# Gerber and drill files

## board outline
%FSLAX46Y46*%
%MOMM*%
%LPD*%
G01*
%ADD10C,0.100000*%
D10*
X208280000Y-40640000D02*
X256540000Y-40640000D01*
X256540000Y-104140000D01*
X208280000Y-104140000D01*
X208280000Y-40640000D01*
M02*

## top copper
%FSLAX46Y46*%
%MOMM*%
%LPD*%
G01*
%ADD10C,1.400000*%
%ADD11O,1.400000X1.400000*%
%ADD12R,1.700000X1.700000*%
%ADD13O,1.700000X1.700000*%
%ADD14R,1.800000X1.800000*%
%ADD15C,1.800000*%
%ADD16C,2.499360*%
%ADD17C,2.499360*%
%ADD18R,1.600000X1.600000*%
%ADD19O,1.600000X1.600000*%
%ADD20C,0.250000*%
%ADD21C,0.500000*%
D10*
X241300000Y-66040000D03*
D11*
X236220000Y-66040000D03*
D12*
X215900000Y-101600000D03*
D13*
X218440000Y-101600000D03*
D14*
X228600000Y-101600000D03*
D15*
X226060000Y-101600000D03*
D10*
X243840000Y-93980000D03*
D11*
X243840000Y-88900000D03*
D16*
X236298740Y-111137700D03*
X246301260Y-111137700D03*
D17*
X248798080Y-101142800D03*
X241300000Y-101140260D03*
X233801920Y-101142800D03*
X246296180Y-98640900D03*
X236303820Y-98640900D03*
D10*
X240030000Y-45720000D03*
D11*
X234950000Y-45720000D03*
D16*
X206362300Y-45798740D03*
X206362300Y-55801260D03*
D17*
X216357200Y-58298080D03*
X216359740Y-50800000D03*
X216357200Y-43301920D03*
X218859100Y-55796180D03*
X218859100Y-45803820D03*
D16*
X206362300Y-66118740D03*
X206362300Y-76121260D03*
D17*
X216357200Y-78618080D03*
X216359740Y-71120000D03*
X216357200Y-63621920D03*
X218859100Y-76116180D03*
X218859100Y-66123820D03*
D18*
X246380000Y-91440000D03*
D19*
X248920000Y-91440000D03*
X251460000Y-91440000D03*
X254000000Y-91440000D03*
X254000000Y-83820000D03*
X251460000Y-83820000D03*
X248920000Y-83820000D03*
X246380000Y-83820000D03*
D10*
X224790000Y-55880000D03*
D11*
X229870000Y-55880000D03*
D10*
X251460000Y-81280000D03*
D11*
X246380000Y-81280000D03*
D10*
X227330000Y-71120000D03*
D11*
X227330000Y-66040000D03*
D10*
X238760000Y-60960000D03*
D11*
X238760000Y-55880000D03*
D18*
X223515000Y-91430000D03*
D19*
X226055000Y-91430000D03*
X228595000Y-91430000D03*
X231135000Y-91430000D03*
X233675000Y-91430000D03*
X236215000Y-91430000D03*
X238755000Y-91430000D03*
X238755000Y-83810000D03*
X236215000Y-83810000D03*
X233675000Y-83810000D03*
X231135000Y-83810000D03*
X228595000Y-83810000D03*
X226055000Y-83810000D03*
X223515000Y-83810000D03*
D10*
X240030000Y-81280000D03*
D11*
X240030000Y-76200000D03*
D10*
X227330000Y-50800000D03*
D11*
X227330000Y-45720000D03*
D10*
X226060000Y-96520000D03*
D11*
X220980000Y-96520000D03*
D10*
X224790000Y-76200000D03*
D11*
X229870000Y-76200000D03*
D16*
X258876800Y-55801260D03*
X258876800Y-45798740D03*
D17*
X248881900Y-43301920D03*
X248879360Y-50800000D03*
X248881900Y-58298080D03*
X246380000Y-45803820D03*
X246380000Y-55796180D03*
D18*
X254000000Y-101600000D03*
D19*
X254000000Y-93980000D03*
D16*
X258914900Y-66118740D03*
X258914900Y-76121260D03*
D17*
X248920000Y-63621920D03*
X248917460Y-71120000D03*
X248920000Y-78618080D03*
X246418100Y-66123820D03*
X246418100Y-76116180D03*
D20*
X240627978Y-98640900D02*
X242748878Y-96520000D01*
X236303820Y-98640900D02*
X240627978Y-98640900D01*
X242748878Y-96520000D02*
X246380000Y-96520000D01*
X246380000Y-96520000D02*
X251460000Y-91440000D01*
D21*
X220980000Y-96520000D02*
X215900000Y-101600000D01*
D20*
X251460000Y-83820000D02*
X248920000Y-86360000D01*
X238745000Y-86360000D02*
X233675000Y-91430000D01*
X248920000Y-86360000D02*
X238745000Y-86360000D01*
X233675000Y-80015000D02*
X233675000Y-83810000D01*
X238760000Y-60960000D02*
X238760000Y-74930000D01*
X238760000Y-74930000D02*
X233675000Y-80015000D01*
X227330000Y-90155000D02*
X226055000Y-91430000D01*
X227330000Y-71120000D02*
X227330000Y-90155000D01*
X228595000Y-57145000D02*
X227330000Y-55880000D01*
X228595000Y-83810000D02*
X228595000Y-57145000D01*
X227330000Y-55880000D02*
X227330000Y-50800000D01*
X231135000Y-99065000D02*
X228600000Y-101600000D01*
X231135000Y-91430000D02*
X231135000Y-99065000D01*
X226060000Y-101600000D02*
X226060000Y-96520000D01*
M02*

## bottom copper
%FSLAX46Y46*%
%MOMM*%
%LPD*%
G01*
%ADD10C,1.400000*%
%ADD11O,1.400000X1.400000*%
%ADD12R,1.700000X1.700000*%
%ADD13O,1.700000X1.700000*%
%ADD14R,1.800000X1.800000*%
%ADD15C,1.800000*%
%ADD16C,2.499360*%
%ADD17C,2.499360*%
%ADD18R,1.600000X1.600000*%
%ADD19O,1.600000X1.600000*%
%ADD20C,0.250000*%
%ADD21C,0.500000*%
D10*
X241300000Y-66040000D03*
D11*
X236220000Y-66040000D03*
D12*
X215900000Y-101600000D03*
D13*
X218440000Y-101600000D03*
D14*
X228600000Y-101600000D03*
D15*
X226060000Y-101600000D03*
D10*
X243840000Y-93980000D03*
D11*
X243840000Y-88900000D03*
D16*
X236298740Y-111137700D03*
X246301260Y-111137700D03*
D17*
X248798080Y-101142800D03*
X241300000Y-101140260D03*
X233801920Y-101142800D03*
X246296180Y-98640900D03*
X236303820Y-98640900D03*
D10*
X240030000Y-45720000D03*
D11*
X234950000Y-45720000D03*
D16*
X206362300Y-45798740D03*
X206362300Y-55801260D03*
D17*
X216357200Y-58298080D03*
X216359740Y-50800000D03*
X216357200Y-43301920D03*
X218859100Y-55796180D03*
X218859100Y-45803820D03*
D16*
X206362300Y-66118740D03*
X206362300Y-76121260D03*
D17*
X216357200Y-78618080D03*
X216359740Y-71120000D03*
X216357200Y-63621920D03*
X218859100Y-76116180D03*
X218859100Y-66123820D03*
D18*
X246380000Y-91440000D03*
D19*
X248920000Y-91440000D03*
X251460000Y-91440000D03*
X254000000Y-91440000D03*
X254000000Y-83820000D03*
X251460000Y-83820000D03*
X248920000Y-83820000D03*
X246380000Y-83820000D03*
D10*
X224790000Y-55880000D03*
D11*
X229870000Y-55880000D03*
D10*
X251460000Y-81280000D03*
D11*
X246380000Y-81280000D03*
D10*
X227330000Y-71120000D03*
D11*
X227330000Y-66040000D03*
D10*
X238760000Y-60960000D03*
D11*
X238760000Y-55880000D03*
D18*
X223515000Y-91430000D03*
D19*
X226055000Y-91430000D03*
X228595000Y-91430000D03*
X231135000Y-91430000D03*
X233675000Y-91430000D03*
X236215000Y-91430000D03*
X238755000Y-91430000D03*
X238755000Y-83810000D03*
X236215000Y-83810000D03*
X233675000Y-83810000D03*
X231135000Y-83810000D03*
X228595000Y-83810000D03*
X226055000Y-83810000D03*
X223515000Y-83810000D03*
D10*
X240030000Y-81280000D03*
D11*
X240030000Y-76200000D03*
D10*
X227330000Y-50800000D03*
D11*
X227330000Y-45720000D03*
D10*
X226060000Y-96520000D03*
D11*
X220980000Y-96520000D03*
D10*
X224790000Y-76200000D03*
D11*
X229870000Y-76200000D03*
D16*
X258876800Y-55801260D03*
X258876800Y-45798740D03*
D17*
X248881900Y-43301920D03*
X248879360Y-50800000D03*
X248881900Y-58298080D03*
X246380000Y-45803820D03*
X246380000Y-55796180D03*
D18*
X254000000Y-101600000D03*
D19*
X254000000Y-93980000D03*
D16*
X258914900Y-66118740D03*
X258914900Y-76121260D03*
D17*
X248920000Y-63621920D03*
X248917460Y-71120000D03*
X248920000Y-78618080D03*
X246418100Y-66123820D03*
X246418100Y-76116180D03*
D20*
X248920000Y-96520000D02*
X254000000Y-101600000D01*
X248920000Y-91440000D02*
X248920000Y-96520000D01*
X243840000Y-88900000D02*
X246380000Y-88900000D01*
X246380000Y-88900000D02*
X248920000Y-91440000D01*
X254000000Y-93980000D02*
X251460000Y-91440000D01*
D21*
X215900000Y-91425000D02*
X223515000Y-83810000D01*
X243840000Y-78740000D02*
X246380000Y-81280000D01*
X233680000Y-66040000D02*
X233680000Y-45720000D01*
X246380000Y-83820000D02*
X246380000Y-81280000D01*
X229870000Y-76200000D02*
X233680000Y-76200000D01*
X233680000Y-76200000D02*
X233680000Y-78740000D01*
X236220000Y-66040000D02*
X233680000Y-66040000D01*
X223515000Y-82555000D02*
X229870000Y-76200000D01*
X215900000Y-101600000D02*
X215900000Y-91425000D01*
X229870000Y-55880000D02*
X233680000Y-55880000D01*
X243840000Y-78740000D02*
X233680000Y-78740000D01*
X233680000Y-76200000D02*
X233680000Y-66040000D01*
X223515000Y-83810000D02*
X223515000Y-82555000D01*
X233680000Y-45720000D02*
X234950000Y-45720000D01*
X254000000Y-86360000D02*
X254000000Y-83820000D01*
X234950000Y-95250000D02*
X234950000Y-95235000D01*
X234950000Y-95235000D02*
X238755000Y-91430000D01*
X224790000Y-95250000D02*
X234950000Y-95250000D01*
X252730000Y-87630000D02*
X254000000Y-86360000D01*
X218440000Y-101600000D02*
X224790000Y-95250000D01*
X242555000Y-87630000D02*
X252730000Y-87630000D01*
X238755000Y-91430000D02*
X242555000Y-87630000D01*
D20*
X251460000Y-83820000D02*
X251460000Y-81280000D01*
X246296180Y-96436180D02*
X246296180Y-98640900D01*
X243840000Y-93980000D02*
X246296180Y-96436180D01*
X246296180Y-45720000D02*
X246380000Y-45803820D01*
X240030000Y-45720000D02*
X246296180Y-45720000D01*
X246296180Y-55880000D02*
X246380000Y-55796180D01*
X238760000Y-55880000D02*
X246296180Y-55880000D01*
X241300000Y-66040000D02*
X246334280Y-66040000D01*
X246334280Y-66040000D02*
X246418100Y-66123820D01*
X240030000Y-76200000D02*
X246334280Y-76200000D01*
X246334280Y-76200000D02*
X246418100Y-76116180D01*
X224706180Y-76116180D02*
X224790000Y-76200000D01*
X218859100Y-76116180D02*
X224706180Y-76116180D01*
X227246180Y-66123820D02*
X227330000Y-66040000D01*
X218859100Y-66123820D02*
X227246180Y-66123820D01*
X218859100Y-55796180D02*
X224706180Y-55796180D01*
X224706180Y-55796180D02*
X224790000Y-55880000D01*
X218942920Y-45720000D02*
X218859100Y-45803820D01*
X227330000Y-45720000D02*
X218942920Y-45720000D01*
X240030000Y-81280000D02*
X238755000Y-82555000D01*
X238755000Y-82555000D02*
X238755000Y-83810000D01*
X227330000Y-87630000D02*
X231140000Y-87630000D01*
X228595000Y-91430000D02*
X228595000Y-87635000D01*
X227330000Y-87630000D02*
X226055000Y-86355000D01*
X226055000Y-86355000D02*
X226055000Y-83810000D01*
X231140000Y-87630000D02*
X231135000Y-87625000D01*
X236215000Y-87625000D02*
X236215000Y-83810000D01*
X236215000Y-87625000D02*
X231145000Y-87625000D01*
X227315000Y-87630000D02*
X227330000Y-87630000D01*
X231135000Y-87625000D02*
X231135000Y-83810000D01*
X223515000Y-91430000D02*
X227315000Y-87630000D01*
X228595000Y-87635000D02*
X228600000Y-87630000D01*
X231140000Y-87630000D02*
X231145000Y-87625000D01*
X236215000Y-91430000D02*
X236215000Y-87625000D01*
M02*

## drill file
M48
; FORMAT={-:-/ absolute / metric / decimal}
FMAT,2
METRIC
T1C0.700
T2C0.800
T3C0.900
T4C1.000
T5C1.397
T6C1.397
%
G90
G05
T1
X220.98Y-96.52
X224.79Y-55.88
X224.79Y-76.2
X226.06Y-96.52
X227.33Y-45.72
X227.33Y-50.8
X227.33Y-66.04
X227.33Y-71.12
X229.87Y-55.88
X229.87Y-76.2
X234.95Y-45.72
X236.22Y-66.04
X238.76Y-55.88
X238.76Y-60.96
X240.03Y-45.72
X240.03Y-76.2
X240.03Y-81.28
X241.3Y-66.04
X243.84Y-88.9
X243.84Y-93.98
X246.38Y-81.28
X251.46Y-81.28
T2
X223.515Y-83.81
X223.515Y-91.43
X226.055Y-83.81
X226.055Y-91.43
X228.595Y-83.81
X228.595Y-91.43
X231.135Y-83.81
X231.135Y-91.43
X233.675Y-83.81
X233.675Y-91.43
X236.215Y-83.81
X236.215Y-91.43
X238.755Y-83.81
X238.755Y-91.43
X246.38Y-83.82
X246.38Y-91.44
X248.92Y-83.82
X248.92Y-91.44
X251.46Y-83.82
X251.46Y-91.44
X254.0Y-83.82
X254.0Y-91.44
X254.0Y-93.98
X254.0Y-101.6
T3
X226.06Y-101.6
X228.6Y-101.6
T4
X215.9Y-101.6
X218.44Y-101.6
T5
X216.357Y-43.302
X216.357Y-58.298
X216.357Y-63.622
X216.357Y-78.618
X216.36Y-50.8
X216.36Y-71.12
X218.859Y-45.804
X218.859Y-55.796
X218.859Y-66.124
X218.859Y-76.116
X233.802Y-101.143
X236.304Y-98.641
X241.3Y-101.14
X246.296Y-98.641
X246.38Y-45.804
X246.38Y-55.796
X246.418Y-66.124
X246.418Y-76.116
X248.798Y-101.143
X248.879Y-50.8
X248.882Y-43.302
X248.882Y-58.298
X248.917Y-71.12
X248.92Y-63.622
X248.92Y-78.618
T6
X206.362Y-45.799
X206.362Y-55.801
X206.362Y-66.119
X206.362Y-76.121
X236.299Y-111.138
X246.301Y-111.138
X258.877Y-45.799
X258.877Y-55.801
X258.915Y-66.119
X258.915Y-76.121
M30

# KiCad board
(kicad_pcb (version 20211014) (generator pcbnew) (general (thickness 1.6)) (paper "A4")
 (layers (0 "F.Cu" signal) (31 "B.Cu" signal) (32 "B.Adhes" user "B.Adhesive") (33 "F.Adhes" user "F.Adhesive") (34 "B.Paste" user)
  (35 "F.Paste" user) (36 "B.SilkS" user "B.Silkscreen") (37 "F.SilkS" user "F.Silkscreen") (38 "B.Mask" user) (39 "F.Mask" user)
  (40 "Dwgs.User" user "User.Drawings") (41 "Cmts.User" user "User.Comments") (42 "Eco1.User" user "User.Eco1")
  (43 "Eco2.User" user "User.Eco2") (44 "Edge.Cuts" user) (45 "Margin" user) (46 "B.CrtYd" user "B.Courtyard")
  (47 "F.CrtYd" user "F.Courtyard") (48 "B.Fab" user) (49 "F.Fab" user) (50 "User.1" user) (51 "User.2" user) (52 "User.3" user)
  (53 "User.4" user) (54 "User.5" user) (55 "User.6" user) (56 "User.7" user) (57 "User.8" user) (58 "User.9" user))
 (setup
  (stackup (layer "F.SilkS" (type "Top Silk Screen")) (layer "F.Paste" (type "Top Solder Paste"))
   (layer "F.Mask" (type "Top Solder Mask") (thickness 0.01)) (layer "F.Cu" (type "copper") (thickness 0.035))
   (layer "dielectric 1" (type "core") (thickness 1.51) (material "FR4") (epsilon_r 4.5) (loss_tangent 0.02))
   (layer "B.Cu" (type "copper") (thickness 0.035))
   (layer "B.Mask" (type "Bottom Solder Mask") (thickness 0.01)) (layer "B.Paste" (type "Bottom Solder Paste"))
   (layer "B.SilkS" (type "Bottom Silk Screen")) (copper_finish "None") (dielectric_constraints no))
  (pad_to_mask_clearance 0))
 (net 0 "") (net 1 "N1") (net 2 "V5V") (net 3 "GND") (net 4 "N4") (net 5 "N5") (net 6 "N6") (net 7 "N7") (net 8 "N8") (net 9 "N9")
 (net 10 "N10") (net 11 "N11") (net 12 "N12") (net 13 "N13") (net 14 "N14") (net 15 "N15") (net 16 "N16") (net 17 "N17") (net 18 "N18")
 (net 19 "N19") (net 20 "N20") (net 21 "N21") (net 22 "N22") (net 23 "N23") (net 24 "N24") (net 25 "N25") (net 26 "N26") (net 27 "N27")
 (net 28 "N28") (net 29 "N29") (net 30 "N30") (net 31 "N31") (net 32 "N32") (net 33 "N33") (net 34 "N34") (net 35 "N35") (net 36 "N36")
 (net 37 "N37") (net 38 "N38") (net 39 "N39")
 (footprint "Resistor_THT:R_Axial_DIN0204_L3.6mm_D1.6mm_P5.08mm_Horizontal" (layer "F.Cu") (at 241.3 66.04 180)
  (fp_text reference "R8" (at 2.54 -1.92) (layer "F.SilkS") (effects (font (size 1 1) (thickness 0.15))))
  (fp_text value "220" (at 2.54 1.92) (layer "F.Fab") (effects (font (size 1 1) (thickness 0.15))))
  (pad "1" thru_hole circle (at 0 0 180) (size 1.4 1.4) (drill 0.7) (layers *.Cu *.Mask) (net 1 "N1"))
  (pad "2" thru_hole oval (at 5.08 0 180) (size 1.4 1.4) (drill 0.7) (layers *.Cu *.Mask) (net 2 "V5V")))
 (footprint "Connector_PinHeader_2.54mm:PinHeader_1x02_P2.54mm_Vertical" (layer "F.Cu") (at 215.9 101.6 90)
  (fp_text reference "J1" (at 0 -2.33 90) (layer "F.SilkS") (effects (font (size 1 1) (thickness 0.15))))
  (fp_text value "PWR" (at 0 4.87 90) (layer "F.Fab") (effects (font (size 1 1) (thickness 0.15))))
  (pad "1" thru_hole rect (at 0 0 90) (size 1.7 1.7) (drill 1) (layers *.Cu *.Mask) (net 2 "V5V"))
  (pad "2" thru_hole oval (at 0 2.54 90) (size 1.7 1.7) (drill 1) (layers *.Cu *.Mask) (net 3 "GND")))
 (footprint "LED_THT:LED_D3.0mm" (layer "F.Cu") (at 228.6 101.6 180)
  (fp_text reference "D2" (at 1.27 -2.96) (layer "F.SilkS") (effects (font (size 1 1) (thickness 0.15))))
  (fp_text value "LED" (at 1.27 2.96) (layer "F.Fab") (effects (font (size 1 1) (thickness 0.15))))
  (pad "1" thru_hole rect (at 0 0 180) (size 1.8 1.8) (drill 0.9) (layers *.Cu *.Mask) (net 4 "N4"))
  (pad "2" thru_hole circle (at 2.54 0 180) (size 1.8 1.8) (drill 0.9) (layers *.Cu *.Mask) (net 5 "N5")))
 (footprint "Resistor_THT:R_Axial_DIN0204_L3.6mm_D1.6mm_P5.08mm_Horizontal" (layer "F.Cu") (at 243.84 93.98 90)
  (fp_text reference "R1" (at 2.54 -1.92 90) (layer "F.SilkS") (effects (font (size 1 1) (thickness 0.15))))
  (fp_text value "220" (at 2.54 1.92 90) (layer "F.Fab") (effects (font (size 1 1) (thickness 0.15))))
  (pad "1" thru_hole circle (at 0 0 90) (size 1.4 1.4) (drill 0.7) (layers *.Cu *.Mask) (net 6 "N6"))
  (pad "2" thru_hole oval (at 5.08 0 90) (size 1.4 1.4) (drill 0.7) (layers *.Cu *.Mask) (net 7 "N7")))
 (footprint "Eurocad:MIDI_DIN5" (layer "F.Cu") (at 241.3 104.14)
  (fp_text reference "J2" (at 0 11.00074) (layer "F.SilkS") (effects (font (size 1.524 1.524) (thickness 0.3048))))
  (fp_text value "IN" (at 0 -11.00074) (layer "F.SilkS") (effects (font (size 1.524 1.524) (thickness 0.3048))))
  (pad "" np_thru_hole circle locked (at -5.00126 6.9977) (size 2.49936 2.49936) (drill 1.397) (layers *.Cu *.Mask "F.SilkS"))
  (pad "" np_thru_hole circle locked (at 5.00126 6.9977) (size 2.49936 2.49936) (drill 1.397) (layers *.Cu *.Mask "F.SilkS"))
  (pad "1" thru_hole circle locked (at 7.49808 -2.9972) (size 2.49936 2.49936) (drill 1.397) (layers *.Cu *.SilkS *.Mask) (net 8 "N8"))
  (pad "2" thru_hole circle locked (at 0 -2.99974) (size 2.49936 2.49936) (drill 1.397) (layers *.Cu *.SilkS *.Mask) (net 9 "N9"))
  (pad "3" thru_hole circle locked (at -7.49808 -2.9972) (size 2.49936 2.49936) (drill 1.397) (layers *.Cu *.SilkS *.Mask) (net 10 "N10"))
  (pad "4" thru_hole circle locked (at 4.99618 -5.4991) (size 2.49936 2.49936) (drill 1.397) (layers *.Cu *.SilkS *.Mask) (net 6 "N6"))
  (pad "5" thru_hole circle locked (at -4.99618 -5.4991) (size 2.49936 2.49936) (drill 1.397) (layers *.Cu *.SilkS *.Mask) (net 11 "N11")))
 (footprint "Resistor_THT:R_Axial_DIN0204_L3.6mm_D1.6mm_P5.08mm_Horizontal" (layer "F.Cu") (at 240.03 45.72 180)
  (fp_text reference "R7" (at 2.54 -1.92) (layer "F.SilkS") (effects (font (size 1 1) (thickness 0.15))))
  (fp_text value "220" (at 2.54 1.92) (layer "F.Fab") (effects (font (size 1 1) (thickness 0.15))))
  (pad "1" thru_hole circle (at 0 0 180) (size 1.4 1.4) (drill 0.7) (layers *.Cu *.Mask) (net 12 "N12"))
  (pad "2" thru_hole oval (at 5.08 0 180) (size 1.4 1.4) (drill 0.7) (layers *.Cu *.Mask) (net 2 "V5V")))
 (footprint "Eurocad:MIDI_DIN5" (layer "F.Cu") (at 213.36 50.8 -90)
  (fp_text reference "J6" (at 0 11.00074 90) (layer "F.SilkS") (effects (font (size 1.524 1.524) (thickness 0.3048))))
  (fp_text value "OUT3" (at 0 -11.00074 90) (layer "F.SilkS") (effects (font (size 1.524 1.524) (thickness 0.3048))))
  (pad "" np_thru_hole circle locked (at -5.00126 6.9977 270) (size 2.49936 2.49936) (drill 1.397) (layers *.Cu *.Mask "F.SilkS"))
  (pad "" np_thru_hole circle locked (at 5.00126 6.9977 270) (size 2.49936 2.49936) (drill 1.397) (layers *.Cu *.Mask "F.SilkS"))
  (pad "1" thru_hole circle locked (at 7.49808 -2.9972 270) (size 2.49936 2.49936) (drill 1.397) (layers *.Cu *.SilkS *.Mask) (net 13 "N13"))
  (pad "2" thru_hole circle locked (at 0 -2.99974 270) (size 2.49936 2.49936) (drill 1.397) (layers *.Cu *.SilkS *.Mask) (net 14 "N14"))
  (pad "3" thru_hole circle locked (at -7.49808 -2.9972 270) (size 2.49936 2.49936) (drill 1.397) (layers *.Cu *.SilkS *.Mask)
   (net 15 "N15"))
  (pad "4" thru_hole circle locked (at 4.99618 -5.4991 270) (size 2.49936 2.49936) (drill 1.397) (layers *.Cu *.SilkS *.Mask) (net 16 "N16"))
  (pad "5" thru_hole circle locked (at -4.99618 -5.4991 270) (size 2.49936 2.49936) (drill 1.397) (layers *.Cu *.SilkS *.Mask)
   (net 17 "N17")))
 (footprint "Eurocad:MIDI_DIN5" (layer "F.Cu") (at 213.36 71.12 -90)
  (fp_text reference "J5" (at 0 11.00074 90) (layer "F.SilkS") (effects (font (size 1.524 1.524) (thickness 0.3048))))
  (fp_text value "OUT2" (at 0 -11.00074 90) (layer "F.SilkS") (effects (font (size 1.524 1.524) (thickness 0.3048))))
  (pad "" np_thru_hole circle locked (at -5.00126 6.9977 270) (size 2.49936 2.49936) (drill 1.397) (layers *.Cu *.Mask "F.SilkS"))
  (pad "" np_thru_hole circle locked (at 5.00126 6.9977 270) (size 2.49936 2.49936) (drill 1.397) (layers *.Cu *.Mask "F.SilkS"))
  (pad "1" thru_hole circle locked (at 7.49808 -2.9972 270) (size 2.49936 2.49936) (drill 1.397) (layers *.Cu *.SilkS *.Mask) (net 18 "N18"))
  (pad "2" thru_hole circle locked (at 0 -2.99974 270) (size 2.49936 2.49936) (drill 1.397) (layers *.Cu *.SilkS *.Mask) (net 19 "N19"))
  (pad "3" thru_hole circle locked (at -7.49808 -2.9972 270) (size 2.49936 2.49936) (drill 1.397) (layers *.Cu *.SilkS *.Mask)
   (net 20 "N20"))
  (pad "4" thru_hole circle locked (at 4.99618 -5.4991 270) (size 2.49936 2.49936) (drill 1.397) (layers *.Cu *.SilkS *.Mask) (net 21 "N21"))
  (pad "5" thru_hole circle locked (at -4.99618 -5.4991 270) (size 2.49936 2.49936) (drill 1.397) (layers *.Cu *.SilkS *.Mask)
   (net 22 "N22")))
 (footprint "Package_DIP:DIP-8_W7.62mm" (layer "F.Cu") (at 246.38 91.44 90)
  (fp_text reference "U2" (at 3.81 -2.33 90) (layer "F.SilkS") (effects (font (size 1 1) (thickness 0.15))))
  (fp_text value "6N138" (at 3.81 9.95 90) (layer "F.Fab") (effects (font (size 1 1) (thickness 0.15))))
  (pad "1" thru_hole rect (at 0 0 90) (size 1.6 1.6) (drill 0.8) (layers *.Cu *.Mask) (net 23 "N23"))
  (pad "2" thru_hole oval (at 0 2.54 90) (size 1.6 1.6) (drill 0.8) (layers *.Cu *.Mask) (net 7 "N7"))
  (pad "3" thru_hole oval (at 0 5.08 90) (size 1.6 1.6) (drill 0.8) (layers *.Cu *.Mask) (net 11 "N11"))
  (pad "4" thru_hole oval (at 0 7.62 90) (size 1.6 1.6) (drill 0.8) (layers *.Cu *.Mask) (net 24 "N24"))
  (pad "5" thru_hole oval (at 7.62 7.62 90) (size 1.6 1.6) (drill 0.8) (layers *.Cu *.Mask) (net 3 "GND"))
  (pad "6" thru_hole oval (at 7.62 5.08 90) (size 1.6 1.6) (drill 0.8) (layers *.Cu *.Mask) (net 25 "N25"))
  (pad "7" thru_hole oval (at 7.62 2.54 90) (size 1.6 1.6) (drill 0.8) (layers *.Cu *.Mask) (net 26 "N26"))
  (pad "8" thru_hole oval (at 7.62 0 90) (size 1.6 1.6) (drill 0.8) (layers *.Cu *.Mask) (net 2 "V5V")))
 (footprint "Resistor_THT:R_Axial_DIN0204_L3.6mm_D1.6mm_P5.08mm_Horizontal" (layer "F.Cu") (at 224.79 55.88)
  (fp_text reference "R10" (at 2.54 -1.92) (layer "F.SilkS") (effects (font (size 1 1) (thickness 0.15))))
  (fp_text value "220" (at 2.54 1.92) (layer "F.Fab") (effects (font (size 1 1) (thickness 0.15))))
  (pad "1" thru_hole circle (at 0 0) (size 1.4 1.4) (drill 0.7) (layers *.Cu *.Mask) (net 16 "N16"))
  (pad "2" thru_hole oval (at 5.08 0) (size 1.4 1.4) (drill 0.7) (layers *.Cu *.Mask) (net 2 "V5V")))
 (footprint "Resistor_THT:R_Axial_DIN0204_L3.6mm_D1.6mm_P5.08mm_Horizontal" (layer "F.Cu") (at 251.46 81.28 180)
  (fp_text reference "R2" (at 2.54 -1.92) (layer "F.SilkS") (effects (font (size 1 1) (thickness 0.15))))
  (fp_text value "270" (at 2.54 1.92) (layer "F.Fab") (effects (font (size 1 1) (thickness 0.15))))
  (pad "1" thru_hole circle (at 0 0 180) (size 1.4 1.4) (drill 0.7) (layers *.Cu *.Mask) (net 25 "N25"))
  (pad "2" thru_hole oval (at 5.08 0 180) (size 1.4 1.4) (drill 0.7) (layers *.Cu *.Mask) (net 2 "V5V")))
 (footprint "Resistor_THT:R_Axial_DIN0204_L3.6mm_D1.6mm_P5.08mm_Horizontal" (layer "F.Cu") (at 227.33 71.12 90)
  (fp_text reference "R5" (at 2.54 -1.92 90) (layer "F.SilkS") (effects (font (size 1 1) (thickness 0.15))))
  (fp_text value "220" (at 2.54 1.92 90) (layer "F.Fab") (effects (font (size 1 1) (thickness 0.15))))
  (pad "1" thru_hole circle (at 0 0 90) (size 1.4 1.4) (drill 0.7) (layers *.Cu *.Mask) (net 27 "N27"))
  (pad "2" thru_hole oval (at 5.08 0 90) (size 1.4 1.4) (drill 0.7) (layers *.Cu *.Mask) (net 22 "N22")))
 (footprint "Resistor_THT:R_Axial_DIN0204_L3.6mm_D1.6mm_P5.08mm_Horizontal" (layer "F.Cu") (at 238.76 60.96 90)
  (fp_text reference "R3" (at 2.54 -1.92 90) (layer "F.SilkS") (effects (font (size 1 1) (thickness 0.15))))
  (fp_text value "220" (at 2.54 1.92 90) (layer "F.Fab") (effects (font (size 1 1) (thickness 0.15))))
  (pad "1" thru_hole circle (at 0 0 90) (size 1.4 1.4) (drill 0.7) (layers *.Cu *.Mask) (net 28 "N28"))
  (pad "2" thru_hole oval (at 5.08 0 90) (size 1.4 1.4) (drill 0.7) (layers *.Cu *.Mask) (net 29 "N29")))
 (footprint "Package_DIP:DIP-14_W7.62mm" (layer "F.Cu") (at 223.515 91.43 90)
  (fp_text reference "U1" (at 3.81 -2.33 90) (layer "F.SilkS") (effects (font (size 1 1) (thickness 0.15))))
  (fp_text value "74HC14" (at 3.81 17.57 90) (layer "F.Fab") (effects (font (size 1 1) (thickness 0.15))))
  (pad "1" thru_hole rect (at 0 0 90) (size 1.6 1.6) (drill 0.8) (layers *.Cu *.Mask) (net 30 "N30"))
  (pad "2" thru_hole oval (at 0 2.54 90) (size 1.6 1.6) (drill 0.8) (layers *.Cu *.Mask) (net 27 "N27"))
  (pad "3" thru_hole oval (at 0 5.08 90) (size 1.6 1.6) (drill 0.8) (layers *.Cu *.Mask) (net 30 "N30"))
  (pad "4" thru_hole oval (at 0 7.62 90) (size 1.6 1.6) (drill 0.8) (layers *.Cu *.Mask) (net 4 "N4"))
  (pad "5" thru_hole oval (at 0 10.16 90) (size 1.6 1.6) (drill 0.8) (layers *.Cu *.Mask) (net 25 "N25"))
  (pad "6" thru_hole oval (at 0 12.7 90) (size 1.6 1.6) (drill 0.8) (layers *.Cu *.Mask) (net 30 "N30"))
  (pad "7" thru_hole oval (at 0 15.24 90) (size 1.6 1.6) (drill 0.8) (layers *.Cu *.Mask) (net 3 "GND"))
  (pad "8" thru_hole oval (at 7.62 15.24 90) (size 1.6 1.6) (drill 0.8) (layers *.Cu *.Mask) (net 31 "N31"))
  (pad "9" thru_hole oval (at 7.62 12.7 90) (size 1.6 1.6) (drill 0.8) (layers *.Cu *.Mask) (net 30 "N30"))
  (pad "10" thru_hole oval (at 7.62 10.16 90) (size 1.6 1.6) (drill 0.8) (layers *.Cu *.Mask) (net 28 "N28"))
  (pad "11" thru_hole oval (at 7.62 7.62 90) (size 1.6 1.6) (drill 0.8) (layers *.Cu *.Mask) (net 30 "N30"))
  (pad "12" thru_hole oval (at 7.62 5.08 90) (size 1.6 1.6) (drill 0.8) (layers *.Cu *.Mask) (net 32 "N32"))
  (pad "13" thru_hole oval (at 7.62 2.54 90) (size 1.6 1.6) (drill 0.8) (layers *.Cu *.Mask) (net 30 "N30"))
  (pad "14" thru_hole oval (at 7.62 0 90) (size 1.6 1.6) (drill 0.8) (layers *.Cu *.Mask) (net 2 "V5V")))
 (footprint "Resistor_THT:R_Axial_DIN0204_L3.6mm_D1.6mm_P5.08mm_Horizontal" (layer "F.Cu") (at 240.03 81.28 90)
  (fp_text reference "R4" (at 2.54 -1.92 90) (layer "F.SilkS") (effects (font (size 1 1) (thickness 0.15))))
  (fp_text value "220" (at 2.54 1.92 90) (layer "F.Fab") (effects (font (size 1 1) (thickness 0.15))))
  (pad "1" thru_hole circle (at 0 0 90) (size 1.4 1.4) (drill 0.7) (layers *.Cu *.Mask) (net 31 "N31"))
  (pad "2" thru_hole oval (at 5.08 0 90) (size 1.4 1.4) (drill 0.7) (layers *.Cu *.Mask) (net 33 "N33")))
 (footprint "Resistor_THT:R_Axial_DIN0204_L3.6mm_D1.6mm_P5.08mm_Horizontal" (layer "F.Cu") (at 227.33 50.8 90)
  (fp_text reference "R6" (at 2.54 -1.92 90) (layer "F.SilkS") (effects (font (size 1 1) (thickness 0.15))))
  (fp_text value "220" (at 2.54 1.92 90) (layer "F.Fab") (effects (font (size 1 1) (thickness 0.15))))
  (pad "1" thru_hole circle (at 0 0 90) (size 1.4 1.4) (drill 0.7) (layers *.Cu *.Mask) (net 32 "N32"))
  (pad "2" thru_hole oval (at 5.08 0 90) (size 1.4 1.4) (drill 0.7) (layers *.Cu *.Mask) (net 17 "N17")))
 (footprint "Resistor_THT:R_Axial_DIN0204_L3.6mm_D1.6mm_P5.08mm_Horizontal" (layer "F.Cu") (at 226.06 96.52 180)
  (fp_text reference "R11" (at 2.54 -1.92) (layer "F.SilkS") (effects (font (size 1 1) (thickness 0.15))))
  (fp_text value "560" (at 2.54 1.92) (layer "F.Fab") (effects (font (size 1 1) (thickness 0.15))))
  (pad "1" thru_hole circle (at 0 0 180) (size 1.4 1.4) (drill 0.7) (layers *.Cu *.Mask) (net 5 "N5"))
  (pad "2" thru_hole oval (at 5.08 0 180) (size 1.4 1.4) (drill 0.7) (layers *.Cu *.Mask) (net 2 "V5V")))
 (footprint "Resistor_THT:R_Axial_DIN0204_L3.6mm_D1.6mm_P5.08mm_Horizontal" (layer "F.Cu") (at 224.79 76.2)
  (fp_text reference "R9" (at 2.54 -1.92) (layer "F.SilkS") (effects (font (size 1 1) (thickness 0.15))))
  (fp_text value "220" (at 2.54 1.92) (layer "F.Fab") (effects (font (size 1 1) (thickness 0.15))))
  (pad "1" thru_hole circle (at 0 0) (size 1.4 1.4) (drill 0.7) (layers *.Cu *.Mask) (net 21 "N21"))
  (pad "2" thru_hole oval (at 5.08 0) (size 1.4 1.4) (drill 0.7) (layers *.Cu *.Mask) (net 2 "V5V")))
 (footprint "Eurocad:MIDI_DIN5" (layer "F.Cu") (at 251.8791 50.8 90)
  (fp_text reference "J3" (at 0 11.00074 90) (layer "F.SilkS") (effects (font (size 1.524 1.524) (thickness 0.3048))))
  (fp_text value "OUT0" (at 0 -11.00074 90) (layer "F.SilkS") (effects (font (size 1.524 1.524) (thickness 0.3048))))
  (pad "" np_thru_hole circle locked (at -5.00126 6.9977 90) (size 2.49936 2.49936) (drill 1.397) (layers *.Cu *.Mask "F.SilkS"))
  (pad "" np_thru_hole circle locked (at 5.00126 6.9977 90) (size 2.49936 2.49936) (drill 1.397) (layers *.Cu *.Mask "F.SilkS"))
  (pad "1" thru_hole circle locked (at 7.49808 -2.9972 90) (size 2.49936 2.49936) (drill 1.397) (layers *.Cu *.SilkS *.Mask) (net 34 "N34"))
  (pad "2" thru_hole circle locked (at 0 -2.99974 90) (size 2.49936 2.49936) (drill 1.397) (layers *.Cu *.SilkS *.Mask) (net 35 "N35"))
  (pad "3" thru_hole circle locked (at -7.49808 -2.9972 90) (size 2.49936 2.49936) (drill 1.397) (layers *.Cu *.SilkS *.Mask) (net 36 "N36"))
  (pad "4" thru_hole circle locked (at 4.99618 -5.4991 90) (size 2.49936 2.49936) (drill 1.397) (layers *.Cu *.SilkS *.Mask) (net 12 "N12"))
  (pad "5" thru_hole circle locked (at -4.99618 -5.4991 90) (size 2.49936 2.49936) (drill 1.397) (layers *.Cu *.SilkS *.Mask) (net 29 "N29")))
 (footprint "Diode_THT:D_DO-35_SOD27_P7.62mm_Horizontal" (layer "F.Cu") (at 254 101.6 90)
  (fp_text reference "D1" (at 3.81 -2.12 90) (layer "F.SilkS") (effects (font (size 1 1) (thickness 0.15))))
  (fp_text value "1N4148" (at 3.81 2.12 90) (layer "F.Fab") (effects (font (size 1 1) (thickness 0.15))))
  (pad "1" thru_hole rect (at 0 0 90) (size 1.6 1.6) (drill 0.8) (layers *.Cu *.Mask) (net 7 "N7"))
  (pad "2" thru_hole oval (at 7.62 0 90) (size 1.6 1.6) (drill 0.8) (layers *.Cu *.Mask) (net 11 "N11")))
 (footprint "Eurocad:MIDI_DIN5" (layer "F.Cu") (at 251.9172 71.12 90)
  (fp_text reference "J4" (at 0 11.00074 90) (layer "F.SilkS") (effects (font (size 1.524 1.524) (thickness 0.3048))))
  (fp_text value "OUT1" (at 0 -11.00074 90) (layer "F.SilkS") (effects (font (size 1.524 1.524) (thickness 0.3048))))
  (pad "" np_thru_hole circle locked (at 5.00126 6.9977 90) (size 2.49936 2.49936) (drill 1.397) (layers *.Cu *.Mask "F.SilkS"))
  (pad "" np_thru_hole circle locked (at -5.00126 6.9977 90) (size 2.49936 2.49936) (drill 1.397) (layers *.Cu *.Mask "F.SilkS"))
  (pad "1" thru_hole circle locked (at 7.49808 -2.9972 90) (size 2.49936 2.49936) (drill 1.397) (layers *.Cu *.SilkS *.Mask) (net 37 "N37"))
  (pad "2" thru_hole circle locked (at 0 -2.99974 90) (size 2.49936 2.49936) (drill 1.397) (layers *.Cu *.SilkS *.Mask) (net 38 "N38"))
  (pad "3" thru_hole circle locked (at -7.49808 -2.9972 90) (size 2.49936 2.49936) (drill 1.397) (layers *.Cu *.SilkS *.Mask) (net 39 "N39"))
  (pad "4" thru_hole circle locked (at 4.99618 -5.4991 90) (size 2.49936 2.49936) (drill 1.397) (layers *.Cu *.SilkS *.Mask) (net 1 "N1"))
  (pad "5" thru_hole circle locked (at -4.99618 -5.4991 90) (size 2.49936 2.49936) (drill 1.397) (layers *.Cu *.SilkS *.Mask) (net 33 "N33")))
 (gr_rect (start 208.28 40.64) (end 256.54 104.14) (layer "Edge.Cuts") (width 0.1) (fill none))
 (segment (start 248.92 96.52) (end 254 101.6) (width 0.25) (layer "B.Cu") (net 7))
 (segment (start 248.92 91.44) (end 248.92 96.52) (width 0.25) (layer "B.Cu") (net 7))
 (segment (start 243.84 88.9) (end 246.38 88.9) (width 0.25) (layer "B.Cu") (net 7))
 (segment (start 246.38 88.9) (end 248.92 91.44) (width 0.25) (layer "B.Cu") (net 7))
 (segment (start 240.627978 98.6409) (end 242.748878 96.52) (width 0.25) (layer "F.Cu") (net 11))
 (segment (start 236.30382 98.6409) (end 240.627978 98.6409) (width 0.25) (layer "F.Cu") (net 11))
 (segment (start 242.748878 96.52) (end 246.38 96.52) (width 0.25) (layer "F.Cu") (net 11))
 (segment (start 246.38 96.52) (end 251.46 91.44) (width 0.25) (layer "F.Cu") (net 11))
 (segment (start 254 93.98) (end 251.46 91.44) (width 0.25) (layer "B.Cu") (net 11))
 (segment (start 220.98 96.52) (end 215.9 101.6) (width 0.5) (layer "F.Cu") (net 2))
 (segment (start 215.9 91.425) (end 223.515 83.81) (width 0.5) (layer "B.Cu") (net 2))
 (segment (start 243.84 78.74) (end 246.38 81.28) (width 0.5) (layer "B.Cu") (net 2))
 (segment (start 233.68 66.04) (end 233.68 45.72) (width 0.5) (layer "B.Cu") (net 2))
 (segment (start 246.38 83.82) (end 246.38 81.28) (width 0.5) (layer "B.Cu") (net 2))
 (segment (start 229.87 76.2) (end 233.68 76.2) (width 0.5) (layer "B.Cu") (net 2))
 (segment (start 233.68 76.2) (end 233.68 78.74) (width 0.5) (layer "B.Cu") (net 2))
 (segment (start 236.22 66.04) (end 233.68 66.04) (width 0.5) (layer "B.Cu") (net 2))
 (segment (start 223.515 82.555) (end 229.87 76.2) (width 0.5) (layer "B.Cu") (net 2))
 (segment (start 215.9 101.6) (end 215.9 91.425) (width 0.5) (layer "B.Cu") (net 2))
 (segment (start 229.87 55.88) (end 233.68 55.88) (width 0.5) (layer "B.Cu") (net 2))
 (segment (start 243.84 78.74) (end 233.68 78.74) (width 0.5) (layer "B.Cu") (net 2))
 (segment (start 233.68 76.2) (end 233.68 66.04) (width 0.5) (layer "B.Cu") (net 2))
 (segment (start 223.515 83.81) (end 223.515 82.555) (width 0.5) (layer "B.Cu") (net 2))
 (segment (start 233.68 45.72) (end 234.95 45.72) (width 0.5) (layer "B.Cu") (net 2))
 (segment (start 254 86.36) (end 254 83.82) (width 0.5) (layer "B.Cu") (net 3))
 (segment (start 234.95 95.25) (end 234.95 95.235) (width 0.5) (layer "B.Cu") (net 3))
 (segment (start 234.95 95.235) (end 238.755 91.43) (width 0.5) (layer "B.Cu") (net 3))
 (segment (start 224.79 95.25) (end 234.95 95.25) (width 0.5) (layer "B.Cu") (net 3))
 (segment (start 252.73 87.63) (end 254 86.36) (width 0.5) (layer "B.Cu") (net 3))
 (segment (start 218.44 101.6) (end 224.79 95.25) (width 0.5) (layer "B.Cu") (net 3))
 (segment (start 242.555 87.63) (end 252.73 87.63) (width 0.5) (layer "B.Cu") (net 3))
 (segment (start 238.755 91.43) (end 242.555 87.63) (width 0.5) (layer "B.Cu") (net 3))
 (segment (start 251.46 83.82) (end 248.92 86.36) (width 0.25) (layer "F.Cu") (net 25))
 (segment (start 238.745 86.36) (end 233.675 91.43) (width 0.25) (layer "F.Cu") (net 25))
 (segment (start 248.92 86.36) (end 238.745 86.36) (width 0.25) (layer "F.Cu") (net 25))
 (segment (start 251.46 83.82) (end 251.46 81.28) (width 0.25) (layer "B.Cu") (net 25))
 (segment (start 246.29618 96.43618) (end 246.29618 98.6409) (width 0.25) (layer "B.Cu") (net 6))
 (segment (start 243.84 93.98) (end 246.29618 96.43618) (width 0.25) (layer "B.Cu") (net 6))
 (segment (start 246.29618 45.72) (end 246.38 45.80382) (width 0.25) (layer "B.Cu") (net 12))
 (segment (start 240.03 45.72) (end 246.29618 45.72) (width 0.25) (layer "B.Cu") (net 12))
 (segment (start 246.29618 55.88) (end 246.38 55.79618) (width 0.25) (layer "B.Cu") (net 29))
 (segment (start 238.76 55.88) (end 246.29618 55.88) (width 0.25) (layer "B.Cu") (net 29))
 (segment (start 241.3 66.04) (end 246.33428 66.04) (width 0.25) (layer "B.Cu") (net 1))
 (segment (start 246.33428 66.04) (end 246.4181 66.12382) (width 0.25) (layer "B.Cu") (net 1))
 (segment (start 240.03 76.2) (end 246.33428 76.2) (width 0.25) (layer "B.Cu") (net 33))
 (segment (start 246.33428 76.2) (end 246.4181 76.11618) (width 0.25) (layer "B.Cu") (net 33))
 (segment (start 224.70618 76.11618) (end 224.79 76.2) (width 0.25) (layer "B.Cu") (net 21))
 (segment (start 218.8591 76.11618) (end 224.70618 76.11618) (width 0.25) (layer "B.Cu") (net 21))
 (segment (start 227.24618 66.12382) (end 227.33 66.04) (width 0.25) (layer "B.Cu") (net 22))
 (segment (start 218.8591 66.12382) (end 227.24618 66.12382) (width 0.25) (layer "B.Cu") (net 22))
 (segment (start 218.8591 55.79618) (end 224.70618 55.79618) (width 0.25) (layer "B.Cu") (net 16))
 (segment (start 224.70618 55.79618) (end 224.79 55.88) (width 0.25) (layer "B.Cu") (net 16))
 (segment (start 218.94292 45.72) (end 218.8591 45.80382) (width 0.25) (layer "B.Cu") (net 17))
 (segment (start 227.33 45.72) (end 218.94292 45.72) (width 0.25) (layer "B.Cu") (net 17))
 (segment (start 240.03 81.28) (end 238.755 82.555) (width 0.25) (layer "B.Cu") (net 31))
 (segment (start 238.755 82.555) (end 238.755 83.81) (width 0.25) (layer "B.Cu") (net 31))
 (segment (start 227.33 87.63) (end 231.14 87.63) (width 0.25) (layer "B.Cu") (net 30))
 (segment (start 228.595 91.43) (end 228.595 87.635) (width 0.25) (layer "B.Cu") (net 30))
 (segment (start 227.33 87.63) (end 226.055 86.355) (width 0.25) (layer "B.Cu") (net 30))
 (segment (start 226.055 86.355) (end 226.055 83.81) (width 0.25) (layer "B.Cu") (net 30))
 (segment (start 231.14 87.63) (end 231.135 87.625) (width 0.25) (layer "B.Cu") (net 30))
 (segment (start 236.215 87.625) (end 236.215 83.81) (width 0.25) (layer "B.Cu") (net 30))
 (segment (start 236.215 87.625) (end 231.145 87.625) (width 0.25) (layer "B.Cu") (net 30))
 (segment (start 227.315 87.63) (end 227.33 87.63) (width 0.25) (layer "B.Cu") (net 30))
 (segment (start 231.135 87.625) (end 231.135 83.81) (width 0.25) (layer "B.Cu") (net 30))
 (segment (start 223.515 91.43) (end 227.315 87.63) (width 0.25) (layer "B.Cu") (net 30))
 (segment (start 228.595 87.635) (end 228.6 87.63) (width 0.25) (layer "B.Cu") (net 30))
 (segment (start 231.14 87.63) (end 231.145 87.625) (width 0.25) (layer "B.Cu") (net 30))
 (segment (start 236.215 91.43) (end 236.215 87.625) (width 0.25) (layer "B.Cu") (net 30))
 (segment (start 233.675 80.015) (end 233.675 83.81) (width 0.25) (layer "F.Cu") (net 28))
 (segment (start 238.76 60.96) (end 238.76 74.93) (width 0.25) (layer "F.Cu") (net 28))
 (segment (start 238.76 74.93) (end 233.675 80.015) (width 0.25) (layer "F.Cu") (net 28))
 (segment (start 227.33 90.155) (end 226.055 91.43) (width 0.25) (layer "F.Cu") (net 27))
 (segment (start 227.33 71.12) (end 227.33 90.155) (width 0.25) (layer "F.Cu") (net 27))
 (segment (start 228.595 57.145) (end 227.33 55.88) (width 0.25) (layer "F.Cu") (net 32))
 (segment (start 228.595 83.81) (end 228.595 57.145) (width 0.25) (layer "F.Cu") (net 32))
 (segment (start 227.33 55.88) (end 227.33 50.8) (width 0.25) (layer "F.Cu") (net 32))
 (segment (start 231.135 99.065) (end 228.6 101.6) (width 0.25) (layer "F.Cu") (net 4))
 (segment (start 231.135 91.43) (end 231.135 99.065) (width 0.25) (layer "F.Cu") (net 4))
 (segment (start 226.06 101.6) (end 226.06 96.52) (width 0.25) (layer "F.Cu") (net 5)))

